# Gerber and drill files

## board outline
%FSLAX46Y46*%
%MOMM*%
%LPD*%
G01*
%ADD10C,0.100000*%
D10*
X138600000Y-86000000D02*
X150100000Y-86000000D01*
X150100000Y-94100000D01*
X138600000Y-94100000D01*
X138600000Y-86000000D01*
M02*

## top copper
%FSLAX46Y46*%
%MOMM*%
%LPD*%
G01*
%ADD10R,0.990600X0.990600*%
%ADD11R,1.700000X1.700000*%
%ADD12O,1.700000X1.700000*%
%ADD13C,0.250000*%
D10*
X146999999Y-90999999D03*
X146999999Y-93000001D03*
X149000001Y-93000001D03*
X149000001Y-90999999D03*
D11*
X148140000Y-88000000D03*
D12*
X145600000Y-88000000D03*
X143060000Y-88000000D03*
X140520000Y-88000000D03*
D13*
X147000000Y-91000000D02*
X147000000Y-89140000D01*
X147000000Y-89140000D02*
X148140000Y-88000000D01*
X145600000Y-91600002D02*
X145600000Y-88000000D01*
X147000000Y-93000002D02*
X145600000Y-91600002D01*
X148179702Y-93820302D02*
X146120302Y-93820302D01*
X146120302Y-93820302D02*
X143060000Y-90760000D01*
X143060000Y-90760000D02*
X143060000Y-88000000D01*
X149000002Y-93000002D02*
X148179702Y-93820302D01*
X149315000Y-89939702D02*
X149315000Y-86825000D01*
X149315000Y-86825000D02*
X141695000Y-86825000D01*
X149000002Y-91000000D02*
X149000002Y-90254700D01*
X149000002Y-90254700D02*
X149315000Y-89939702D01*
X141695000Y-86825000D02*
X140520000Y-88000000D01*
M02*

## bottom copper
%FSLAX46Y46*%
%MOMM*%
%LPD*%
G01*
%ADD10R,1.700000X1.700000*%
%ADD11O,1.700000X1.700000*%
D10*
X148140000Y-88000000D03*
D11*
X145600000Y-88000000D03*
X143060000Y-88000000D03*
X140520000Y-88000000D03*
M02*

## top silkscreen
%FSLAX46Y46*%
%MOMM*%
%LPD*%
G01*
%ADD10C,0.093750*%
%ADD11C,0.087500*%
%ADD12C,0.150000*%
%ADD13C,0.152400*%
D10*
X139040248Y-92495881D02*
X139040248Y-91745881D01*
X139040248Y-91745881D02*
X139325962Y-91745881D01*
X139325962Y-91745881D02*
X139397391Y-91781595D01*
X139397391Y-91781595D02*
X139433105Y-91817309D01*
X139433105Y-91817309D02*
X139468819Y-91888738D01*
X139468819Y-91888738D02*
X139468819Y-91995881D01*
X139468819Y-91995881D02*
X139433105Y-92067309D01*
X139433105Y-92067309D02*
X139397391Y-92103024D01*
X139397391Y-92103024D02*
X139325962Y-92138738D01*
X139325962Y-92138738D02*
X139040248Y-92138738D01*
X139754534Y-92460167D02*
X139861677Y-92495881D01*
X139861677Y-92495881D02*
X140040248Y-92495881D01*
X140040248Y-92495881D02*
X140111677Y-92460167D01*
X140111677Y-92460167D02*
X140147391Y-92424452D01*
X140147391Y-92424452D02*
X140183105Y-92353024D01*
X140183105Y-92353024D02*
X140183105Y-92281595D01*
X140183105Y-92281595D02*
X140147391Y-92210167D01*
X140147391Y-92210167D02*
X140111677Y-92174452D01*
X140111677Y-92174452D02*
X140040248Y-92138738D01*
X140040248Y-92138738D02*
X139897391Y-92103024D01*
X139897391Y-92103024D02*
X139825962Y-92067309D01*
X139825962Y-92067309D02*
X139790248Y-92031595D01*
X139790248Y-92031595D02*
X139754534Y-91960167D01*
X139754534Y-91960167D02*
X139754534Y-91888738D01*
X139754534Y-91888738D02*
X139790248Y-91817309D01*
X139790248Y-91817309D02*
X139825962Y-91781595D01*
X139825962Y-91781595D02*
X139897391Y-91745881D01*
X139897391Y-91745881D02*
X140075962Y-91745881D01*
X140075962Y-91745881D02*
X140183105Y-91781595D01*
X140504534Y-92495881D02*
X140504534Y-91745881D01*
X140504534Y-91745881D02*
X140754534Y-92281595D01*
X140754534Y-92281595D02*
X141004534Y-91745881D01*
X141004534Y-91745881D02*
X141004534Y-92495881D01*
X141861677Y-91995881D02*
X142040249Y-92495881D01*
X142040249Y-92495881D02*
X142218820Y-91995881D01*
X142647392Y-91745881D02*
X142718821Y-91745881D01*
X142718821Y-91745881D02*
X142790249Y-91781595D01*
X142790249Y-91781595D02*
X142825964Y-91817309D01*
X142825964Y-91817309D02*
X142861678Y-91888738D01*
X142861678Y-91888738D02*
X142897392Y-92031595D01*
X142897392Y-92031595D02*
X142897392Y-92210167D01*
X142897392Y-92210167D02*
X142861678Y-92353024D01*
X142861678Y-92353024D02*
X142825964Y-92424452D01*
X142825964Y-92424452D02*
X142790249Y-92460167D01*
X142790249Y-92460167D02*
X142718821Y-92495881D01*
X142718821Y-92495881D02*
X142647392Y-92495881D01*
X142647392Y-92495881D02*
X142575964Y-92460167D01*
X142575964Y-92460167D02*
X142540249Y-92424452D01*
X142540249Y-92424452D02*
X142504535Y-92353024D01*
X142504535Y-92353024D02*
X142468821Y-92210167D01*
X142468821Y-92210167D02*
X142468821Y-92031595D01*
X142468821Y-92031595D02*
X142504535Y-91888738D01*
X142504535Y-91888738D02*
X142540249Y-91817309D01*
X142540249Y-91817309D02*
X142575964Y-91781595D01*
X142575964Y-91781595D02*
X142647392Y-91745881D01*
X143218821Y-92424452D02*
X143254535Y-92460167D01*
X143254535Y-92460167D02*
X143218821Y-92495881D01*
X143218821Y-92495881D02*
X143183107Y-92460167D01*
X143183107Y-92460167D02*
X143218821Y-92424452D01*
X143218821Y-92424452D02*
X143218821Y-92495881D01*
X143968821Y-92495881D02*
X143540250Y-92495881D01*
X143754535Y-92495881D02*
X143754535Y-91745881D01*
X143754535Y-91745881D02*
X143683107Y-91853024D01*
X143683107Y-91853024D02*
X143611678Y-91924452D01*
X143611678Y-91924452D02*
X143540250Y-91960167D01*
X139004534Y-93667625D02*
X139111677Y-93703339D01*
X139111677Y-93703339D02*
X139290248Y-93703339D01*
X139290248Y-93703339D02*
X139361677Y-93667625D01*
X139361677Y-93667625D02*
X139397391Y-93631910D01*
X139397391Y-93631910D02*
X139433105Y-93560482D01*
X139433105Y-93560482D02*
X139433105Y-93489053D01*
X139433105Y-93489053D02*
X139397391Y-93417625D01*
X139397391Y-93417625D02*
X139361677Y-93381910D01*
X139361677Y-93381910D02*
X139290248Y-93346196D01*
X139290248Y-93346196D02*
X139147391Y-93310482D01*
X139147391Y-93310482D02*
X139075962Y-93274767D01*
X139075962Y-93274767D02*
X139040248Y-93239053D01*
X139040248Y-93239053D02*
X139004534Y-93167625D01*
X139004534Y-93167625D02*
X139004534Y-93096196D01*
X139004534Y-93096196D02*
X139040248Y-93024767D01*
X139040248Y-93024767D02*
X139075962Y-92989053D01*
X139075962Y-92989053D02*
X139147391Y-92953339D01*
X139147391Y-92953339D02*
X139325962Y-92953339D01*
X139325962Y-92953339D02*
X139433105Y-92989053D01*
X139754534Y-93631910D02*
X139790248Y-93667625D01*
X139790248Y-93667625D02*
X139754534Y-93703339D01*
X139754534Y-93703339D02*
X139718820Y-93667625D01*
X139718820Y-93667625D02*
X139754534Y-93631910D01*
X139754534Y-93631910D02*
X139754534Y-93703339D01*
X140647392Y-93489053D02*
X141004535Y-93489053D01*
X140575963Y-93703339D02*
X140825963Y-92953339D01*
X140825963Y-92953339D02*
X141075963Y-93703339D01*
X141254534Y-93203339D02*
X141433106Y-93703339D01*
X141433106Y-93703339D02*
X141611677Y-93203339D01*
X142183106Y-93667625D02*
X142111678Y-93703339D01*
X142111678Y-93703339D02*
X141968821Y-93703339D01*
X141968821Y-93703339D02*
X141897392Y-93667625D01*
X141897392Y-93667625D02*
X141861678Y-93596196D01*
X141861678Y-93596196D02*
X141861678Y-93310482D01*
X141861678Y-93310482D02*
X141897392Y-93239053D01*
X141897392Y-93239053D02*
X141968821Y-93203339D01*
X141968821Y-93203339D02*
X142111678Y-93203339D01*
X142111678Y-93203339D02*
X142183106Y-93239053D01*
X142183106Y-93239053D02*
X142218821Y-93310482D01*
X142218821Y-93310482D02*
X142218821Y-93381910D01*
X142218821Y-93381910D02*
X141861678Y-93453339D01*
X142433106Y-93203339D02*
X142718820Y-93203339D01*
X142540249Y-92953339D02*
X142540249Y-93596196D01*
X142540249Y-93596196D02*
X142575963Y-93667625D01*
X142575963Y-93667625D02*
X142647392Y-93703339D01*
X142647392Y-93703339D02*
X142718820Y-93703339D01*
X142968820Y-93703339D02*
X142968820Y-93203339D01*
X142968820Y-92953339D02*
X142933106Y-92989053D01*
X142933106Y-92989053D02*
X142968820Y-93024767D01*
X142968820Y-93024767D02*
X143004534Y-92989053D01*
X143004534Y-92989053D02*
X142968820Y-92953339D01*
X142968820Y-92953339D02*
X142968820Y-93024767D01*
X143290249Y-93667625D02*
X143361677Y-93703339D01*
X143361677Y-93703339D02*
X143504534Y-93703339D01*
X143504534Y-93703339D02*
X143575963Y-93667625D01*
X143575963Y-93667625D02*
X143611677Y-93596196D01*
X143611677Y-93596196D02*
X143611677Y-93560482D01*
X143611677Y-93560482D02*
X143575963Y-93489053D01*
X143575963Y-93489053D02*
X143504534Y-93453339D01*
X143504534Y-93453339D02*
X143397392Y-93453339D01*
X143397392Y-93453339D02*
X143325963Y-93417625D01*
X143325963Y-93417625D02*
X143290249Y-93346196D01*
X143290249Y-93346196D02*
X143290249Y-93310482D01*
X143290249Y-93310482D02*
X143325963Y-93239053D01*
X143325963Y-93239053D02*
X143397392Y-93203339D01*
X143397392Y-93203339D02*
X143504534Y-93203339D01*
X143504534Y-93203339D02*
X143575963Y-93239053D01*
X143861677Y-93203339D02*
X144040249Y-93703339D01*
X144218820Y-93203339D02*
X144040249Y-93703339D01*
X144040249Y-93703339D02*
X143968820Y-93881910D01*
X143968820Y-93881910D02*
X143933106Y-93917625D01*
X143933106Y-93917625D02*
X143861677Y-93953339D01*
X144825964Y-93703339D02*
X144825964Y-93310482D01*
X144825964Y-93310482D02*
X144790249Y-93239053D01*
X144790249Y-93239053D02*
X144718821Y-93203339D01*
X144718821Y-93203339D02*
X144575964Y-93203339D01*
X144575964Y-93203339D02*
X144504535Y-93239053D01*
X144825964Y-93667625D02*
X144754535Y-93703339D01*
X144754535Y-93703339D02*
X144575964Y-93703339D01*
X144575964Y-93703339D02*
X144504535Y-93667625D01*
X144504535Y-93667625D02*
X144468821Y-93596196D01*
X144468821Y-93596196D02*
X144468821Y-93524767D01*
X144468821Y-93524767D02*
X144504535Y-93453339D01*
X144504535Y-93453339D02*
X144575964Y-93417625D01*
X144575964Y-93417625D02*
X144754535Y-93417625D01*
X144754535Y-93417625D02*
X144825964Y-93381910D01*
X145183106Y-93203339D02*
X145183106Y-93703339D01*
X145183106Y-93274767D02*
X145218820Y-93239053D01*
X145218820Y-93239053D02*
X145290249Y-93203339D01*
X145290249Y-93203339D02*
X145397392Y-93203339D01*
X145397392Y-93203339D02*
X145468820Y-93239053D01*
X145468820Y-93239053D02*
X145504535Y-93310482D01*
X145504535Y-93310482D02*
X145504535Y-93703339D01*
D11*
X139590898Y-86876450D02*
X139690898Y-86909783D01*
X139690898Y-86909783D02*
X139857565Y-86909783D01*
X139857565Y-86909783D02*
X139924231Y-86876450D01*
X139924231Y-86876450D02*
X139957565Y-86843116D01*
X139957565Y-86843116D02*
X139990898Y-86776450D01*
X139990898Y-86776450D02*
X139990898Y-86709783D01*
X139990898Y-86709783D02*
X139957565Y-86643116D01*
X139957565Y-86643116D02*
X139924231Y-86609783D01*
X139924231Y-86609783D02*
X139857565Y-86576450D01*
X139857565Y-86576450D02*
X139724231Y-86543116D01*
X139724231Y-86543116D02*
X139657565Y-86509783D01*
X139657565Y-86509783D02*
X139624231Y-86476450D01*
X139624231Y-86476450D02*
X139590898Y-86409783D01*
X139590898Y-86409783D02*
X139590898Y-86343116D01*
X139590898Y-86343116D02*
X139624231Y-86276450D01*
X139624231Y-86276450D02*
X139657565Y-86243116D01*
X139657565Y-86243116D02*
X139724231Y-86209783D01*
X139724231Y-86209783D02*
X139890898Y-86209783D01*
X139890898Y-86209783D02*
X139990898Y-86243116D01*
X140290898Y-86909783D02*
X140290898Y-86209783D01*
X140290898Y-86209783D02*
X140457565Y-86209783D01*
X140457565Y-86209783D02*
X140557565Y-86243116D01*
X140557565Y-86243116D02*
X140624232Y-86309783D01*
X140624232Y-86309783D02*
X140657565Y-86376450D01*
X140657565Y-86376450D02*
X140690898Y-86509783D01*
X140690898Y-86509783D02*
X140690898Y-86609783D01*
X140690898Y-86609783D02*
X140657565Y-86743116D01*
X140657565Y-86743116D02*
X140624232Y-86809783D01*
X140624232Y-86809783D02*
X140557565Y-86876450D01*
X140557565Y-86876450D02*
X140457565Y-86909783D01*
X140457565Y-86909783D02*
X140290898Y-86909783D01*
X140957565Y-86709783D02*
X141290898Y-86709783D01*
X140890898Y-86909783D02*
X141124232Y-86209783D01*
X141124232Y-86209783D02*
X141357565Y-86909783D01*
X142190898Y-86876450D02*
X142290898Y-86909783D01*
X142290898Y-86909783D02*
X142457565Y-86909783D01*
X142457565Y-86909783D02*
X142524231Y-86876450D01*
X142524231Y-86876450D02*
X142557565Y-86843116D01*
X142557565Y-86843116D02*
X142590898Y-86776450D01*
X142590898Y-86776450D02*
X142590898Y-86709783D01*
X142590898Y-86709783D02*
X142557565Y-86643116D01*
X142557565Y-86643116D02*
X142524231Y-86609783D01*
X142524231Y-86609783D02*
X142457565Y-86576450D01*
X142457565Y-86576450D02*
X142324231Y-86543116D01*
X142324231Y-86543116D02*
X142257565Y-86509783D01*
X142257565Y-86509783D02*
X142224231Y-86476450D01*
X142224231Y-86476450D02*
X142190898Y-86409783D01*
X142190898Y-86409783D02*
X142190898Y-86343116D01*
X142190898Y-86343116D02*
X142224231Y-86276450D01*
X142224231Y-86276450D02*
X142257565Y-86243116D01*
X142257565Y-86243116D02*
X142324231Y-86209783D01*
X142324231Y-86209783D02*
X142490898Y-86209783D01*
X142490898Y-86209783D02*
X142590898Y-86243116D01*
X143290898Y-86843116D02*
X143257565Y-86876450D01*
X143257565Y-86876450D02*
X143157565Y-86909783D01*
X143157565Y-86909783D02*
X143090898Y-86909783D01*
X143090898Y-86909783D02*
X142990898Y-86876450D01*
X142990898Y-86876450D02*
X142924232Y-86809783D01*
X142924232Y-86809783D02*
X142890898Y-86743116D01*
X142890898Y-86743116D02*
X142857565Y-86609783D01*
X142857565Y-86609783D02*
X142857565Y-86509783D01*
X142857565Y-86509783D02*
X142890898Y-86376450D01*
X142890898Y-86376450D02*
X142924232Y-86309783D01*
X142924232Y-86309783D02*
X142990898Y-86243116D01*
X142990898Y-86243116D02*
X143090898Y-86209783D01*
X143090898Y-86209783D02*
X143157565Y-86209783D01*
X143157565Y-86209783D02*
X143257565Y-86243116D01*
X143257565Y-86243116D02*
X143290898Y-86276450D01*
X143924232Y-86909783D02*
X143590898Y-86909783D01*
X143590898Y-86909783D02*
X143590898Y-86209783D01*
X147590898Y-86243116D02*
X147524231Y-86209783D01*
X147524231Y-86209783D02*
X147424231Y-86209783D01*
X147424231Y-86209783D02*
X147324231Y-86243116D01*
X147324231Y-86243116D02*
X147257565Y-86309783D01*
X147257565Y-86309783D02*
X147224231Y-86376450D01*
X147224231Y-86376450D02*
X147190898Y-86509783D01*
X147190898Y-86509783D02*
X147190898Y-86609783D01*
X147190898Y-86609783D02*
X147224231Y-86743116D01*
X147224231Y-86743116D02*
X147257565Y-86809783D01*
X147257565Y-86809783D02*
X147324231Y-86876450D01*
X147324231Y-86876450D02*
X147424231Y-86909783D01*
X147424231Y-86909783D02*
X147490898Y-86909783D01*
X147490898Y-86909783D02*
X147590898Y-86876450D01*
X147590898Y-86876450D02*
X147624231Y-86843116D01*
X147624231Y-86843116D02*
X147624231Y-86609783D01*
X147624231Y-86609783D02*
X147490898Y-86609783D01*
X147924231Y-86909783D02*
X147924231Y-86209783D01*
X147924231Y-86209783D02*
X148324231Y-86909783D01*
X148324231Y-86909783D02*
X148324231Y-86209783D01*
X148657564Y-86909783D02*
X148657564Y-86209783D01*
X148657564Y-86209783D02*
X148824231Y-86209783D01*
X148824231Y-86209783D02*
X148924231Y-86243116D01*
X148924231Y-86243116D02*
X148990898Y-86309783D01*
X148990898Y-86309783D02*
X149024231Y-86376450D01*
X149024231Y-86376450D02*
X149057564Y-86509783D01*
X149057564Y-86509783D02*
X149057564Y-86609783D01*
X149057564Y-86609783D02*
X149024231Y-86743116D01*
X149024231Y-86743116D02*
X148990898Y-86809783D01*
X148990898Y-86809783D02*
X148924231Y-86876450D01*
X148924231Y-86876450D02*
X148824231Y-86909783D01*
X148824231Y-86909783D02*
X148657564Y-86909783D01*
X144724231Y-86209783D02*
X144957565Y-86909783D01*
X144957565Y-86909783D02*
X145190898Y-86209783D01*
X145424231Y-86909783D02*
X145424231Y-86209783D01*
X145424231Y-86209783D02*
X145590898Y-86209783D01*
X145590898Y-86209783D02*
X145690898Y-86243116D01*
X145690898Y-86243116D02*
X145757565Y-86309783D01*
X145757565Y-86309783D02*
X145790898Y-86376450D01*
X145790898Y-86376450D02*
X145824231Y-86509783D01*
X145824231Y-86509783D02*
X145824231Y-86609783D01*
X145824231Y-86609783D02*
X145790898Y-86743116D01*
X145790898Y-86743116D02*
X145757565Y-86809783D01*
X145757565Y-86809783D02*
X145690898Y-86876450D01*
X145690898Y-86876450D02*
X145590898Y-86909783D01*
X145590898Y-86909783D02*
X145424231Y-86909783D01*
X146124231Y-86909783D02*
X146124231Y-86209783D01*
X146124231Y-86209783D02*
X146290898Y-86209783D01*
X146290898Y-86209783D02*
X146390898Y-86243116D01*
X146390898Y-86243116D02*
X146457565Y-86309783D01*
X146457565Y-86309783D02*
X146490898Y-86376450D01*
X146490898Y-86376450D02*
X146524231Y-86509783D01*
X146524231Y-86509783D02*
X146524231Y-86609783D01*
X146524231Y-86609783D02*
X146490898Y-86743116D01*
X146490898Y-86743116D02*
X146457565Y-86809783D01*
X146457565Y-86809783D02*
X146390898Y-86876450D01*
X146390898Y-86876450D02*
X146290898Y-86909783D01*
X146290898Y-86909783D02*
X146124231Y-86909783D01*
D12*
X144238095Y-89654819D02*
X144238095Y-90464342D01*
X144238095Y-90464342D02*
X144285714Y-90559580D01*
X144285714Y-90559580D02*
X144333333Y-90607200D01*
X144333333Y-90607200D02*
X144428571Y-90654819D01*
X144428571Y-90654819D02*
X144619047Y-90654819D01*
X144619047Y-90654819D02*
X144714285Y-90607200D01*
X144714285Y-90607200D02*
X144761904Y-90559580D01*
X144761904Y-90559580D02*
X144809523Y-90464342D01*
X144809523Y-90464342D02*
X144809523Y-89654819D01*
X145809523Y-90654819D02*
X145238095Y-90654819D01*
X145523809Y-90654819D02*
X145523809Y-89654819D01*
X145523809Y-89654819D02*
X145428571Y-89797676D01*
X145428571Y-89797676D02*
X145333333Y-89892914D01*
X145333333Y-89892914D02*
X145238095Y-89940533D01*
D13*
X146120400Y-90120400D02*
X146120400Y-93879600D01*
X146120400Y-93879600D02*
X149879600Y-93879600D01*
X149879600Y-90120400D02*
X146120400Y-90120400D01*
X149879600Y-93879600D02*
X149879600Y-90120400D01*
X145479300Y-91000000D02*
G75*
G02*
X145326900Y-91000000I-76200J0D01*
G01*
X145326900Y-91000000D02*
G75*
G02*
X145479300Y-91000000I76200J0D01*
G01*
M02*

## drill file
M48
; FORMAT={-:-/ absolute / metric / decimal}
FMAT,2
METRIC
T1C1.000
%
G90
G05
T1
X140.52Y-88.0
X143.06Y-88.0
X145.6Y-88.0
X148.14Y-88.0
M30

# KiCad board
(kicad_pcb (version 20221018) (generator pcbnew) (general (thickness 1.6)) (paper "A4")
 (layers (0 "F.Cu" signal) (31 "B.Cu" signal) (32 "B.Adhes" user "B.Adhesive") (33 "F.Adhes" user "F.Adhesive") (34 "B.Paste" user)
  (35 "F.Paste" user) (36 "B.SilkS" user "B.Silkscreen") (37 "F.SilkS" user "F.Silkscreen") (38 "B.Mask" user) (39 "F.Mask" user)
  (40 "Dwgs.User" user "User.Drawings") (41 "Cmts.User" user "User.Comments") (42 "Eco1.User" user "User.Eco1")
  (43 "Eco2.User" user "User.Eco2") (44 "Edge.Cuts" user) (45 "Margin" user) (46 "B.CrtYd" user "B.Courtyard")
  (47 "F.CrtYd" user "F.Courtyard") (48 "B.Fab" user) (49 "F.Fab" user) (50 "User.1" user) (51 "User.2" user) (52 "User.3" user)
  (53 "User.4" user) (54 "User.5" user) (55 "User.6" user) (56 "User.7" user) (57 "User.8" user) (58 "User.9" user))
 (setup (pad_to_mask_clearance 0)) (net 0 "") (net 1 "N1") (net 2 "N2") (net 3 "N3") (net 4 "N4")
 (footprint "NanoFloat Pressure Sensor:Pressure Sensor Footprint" (layer "F.Cu") (at 148 92)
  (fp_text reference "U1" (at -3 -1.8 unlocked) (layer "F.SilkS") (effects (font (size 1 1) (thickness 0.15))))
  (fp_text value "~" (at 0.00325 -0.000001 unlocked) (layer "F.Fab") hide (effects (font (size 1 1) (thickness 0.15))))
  (fp_line (start -1.8796 -1.8796) (end -1.8796 1.8796) (stroke (width 0.1524) (type solid)) (layer "F.SilkS"))
  (fp_line (start -1.8796 1.8796) (end 1.8796 1.8796) (stroke (width 0.1524) (type solid)) (layer "F.SilkS"))
  (fp_line (start 1.8796 -1.8796) (end -1.8796 -1.8796) (stroke (width 0.1524) (type solid)) (layer "F.SilkS"))
  (fp_line (start 1.8796 1.8796) (end 1.8796 -1.8796) (stroke (width 0.1524) (type solid)) (layer "F.SilkS"))
  (fp_circle (center -2.5969 -1) (end -2.5207 -1) (stroke (width 0.1524) (type solid)) (fill none) (layer "F.SilkS"))
  (pad "1" smd rect (at -1.000001 -1.000001) (size 0.9906 0.9906) (layers "F.Cu" "F.Paste" "F.Mask") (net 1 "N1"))
  (pad "2" smd rect (at -1.000001 1.000001) (size 0.9906 0.9906) (layers "F.Cu" "F.Paste" "F.Mask") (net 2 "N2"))
  (pad "3" smd rect (at 1.000001 1.000001) (size 0.9906 0.9906) (layers "F.Cu" "F.Paste" "F.Mask") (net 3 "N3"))
  (pad "4" smd rect (at 1.000001 -1.000001) (size 0.9906 0.9906) (layers "F.Cu" "F.Paste" "F.Mask") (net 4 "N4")))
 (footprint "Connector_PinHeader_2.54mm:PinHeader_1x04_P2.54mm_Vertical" (layer "B.Cu") (at 148.14 88 90)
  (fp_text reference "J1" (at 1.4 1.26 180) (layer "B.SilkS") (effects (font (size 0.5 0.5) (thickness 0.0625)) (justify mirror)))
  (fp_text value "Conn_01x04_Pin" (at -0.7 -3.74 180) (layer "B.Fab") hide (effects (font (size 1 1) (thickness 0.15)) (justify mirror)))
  (pad "1" thru_hole rect (at 0 0 90) (size 1.7 1.7) (drill 1) (layers "*.Cu" "*.Mask") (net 1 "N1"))
  (pad "2" thru_hole oval (at 0 -2.54 90) (size 1.7 1.7) (drill 1) (layers "*.Cu" "*.Mask") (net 2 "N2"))
  (pad "3" thru_hole oval (at 0 -5.08 90) (size 1.7 1.7) (drill 1) (layers "*.Cu" "*.Mask") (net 3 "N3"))
  (pad "4" thru_hole oval (at 0 -7.62 90) (size 1.7 1.7) (drill 1) (layers "*.Cu" "*.Mask") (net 4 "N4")))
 (gr_rect (start 138.6 86) (end 150.1 94.1) (stroke (width 0.1) (type default)) (fill none) (layer "Edge.Cuts"))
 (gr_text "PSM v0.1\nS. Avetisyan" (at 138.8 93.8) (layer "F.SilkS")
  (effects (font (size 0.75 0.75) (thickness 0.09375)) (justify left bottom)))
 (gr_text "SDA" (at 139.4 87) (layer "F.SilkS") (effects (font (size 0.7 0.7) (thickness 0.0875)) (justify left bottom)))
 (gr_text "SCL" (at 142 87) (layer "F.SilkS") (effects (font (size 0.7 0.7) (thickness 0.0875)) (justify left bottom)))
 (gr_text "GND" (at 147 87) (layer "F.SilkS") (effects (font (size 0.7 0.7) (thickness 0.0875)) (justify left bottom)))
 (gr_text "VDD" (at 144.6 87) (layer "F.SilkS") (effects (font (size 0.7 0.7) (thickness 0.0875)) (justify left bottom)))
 (segment (start 147 91) (end 147 89.14) (width 0.25) (layer "F.Cu") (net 1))
 (segment (start 147 89.14) (end 148.14 88) (width 0.25) (layer "F.Cu") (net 1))
 (segment (start 145.6 91.600002) (end 145.6 88) (width 0.25) (layer "F.Cu") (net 2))
 (segment (start 147 93.000002) (end 145.6 91.600002) (width 0.25) (layer "F.Cu") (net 2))
 (segment (start 148.179702 93.820302) (end 146.120302 93.820302) (width 0.25) (layer "F.Cu") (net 3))
 (segment (start 146.120302 93.820302) (end 143.06 90.76) (width 0.25) (layer "F.Cu") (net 3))
 (segment (start 143.06 90.76) (end 143.06 88) (width 0.25) (layer "F.Cu") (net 3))
 (segment (start 149.000002 93.000002) (end 148.179702 93.820302) (width 0.25) (layer "F.Cu") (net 3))
 (segment (start 149.315 89.939702) (end 149.315 86.825) (width 0.25) (layer "F.Cu") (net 4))
 (segment (start 149.315 86.825) (end 141.695 86.825) (width 0.25) (layer "F.Cu") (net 4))
 (segment (start 149.000002 91) (end 149.000002 90.2547) (width 0.25) (layer "F.Cu") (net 4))
 (segment (start 149.000002 90.2547) (end 149.315 89.939702) (width 0.25) (layer "F.Cu") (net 4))
 (segment (start 141.695 86.825) (end 140.52 88) (width 0.25) (layer "F.Cu") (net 4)))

